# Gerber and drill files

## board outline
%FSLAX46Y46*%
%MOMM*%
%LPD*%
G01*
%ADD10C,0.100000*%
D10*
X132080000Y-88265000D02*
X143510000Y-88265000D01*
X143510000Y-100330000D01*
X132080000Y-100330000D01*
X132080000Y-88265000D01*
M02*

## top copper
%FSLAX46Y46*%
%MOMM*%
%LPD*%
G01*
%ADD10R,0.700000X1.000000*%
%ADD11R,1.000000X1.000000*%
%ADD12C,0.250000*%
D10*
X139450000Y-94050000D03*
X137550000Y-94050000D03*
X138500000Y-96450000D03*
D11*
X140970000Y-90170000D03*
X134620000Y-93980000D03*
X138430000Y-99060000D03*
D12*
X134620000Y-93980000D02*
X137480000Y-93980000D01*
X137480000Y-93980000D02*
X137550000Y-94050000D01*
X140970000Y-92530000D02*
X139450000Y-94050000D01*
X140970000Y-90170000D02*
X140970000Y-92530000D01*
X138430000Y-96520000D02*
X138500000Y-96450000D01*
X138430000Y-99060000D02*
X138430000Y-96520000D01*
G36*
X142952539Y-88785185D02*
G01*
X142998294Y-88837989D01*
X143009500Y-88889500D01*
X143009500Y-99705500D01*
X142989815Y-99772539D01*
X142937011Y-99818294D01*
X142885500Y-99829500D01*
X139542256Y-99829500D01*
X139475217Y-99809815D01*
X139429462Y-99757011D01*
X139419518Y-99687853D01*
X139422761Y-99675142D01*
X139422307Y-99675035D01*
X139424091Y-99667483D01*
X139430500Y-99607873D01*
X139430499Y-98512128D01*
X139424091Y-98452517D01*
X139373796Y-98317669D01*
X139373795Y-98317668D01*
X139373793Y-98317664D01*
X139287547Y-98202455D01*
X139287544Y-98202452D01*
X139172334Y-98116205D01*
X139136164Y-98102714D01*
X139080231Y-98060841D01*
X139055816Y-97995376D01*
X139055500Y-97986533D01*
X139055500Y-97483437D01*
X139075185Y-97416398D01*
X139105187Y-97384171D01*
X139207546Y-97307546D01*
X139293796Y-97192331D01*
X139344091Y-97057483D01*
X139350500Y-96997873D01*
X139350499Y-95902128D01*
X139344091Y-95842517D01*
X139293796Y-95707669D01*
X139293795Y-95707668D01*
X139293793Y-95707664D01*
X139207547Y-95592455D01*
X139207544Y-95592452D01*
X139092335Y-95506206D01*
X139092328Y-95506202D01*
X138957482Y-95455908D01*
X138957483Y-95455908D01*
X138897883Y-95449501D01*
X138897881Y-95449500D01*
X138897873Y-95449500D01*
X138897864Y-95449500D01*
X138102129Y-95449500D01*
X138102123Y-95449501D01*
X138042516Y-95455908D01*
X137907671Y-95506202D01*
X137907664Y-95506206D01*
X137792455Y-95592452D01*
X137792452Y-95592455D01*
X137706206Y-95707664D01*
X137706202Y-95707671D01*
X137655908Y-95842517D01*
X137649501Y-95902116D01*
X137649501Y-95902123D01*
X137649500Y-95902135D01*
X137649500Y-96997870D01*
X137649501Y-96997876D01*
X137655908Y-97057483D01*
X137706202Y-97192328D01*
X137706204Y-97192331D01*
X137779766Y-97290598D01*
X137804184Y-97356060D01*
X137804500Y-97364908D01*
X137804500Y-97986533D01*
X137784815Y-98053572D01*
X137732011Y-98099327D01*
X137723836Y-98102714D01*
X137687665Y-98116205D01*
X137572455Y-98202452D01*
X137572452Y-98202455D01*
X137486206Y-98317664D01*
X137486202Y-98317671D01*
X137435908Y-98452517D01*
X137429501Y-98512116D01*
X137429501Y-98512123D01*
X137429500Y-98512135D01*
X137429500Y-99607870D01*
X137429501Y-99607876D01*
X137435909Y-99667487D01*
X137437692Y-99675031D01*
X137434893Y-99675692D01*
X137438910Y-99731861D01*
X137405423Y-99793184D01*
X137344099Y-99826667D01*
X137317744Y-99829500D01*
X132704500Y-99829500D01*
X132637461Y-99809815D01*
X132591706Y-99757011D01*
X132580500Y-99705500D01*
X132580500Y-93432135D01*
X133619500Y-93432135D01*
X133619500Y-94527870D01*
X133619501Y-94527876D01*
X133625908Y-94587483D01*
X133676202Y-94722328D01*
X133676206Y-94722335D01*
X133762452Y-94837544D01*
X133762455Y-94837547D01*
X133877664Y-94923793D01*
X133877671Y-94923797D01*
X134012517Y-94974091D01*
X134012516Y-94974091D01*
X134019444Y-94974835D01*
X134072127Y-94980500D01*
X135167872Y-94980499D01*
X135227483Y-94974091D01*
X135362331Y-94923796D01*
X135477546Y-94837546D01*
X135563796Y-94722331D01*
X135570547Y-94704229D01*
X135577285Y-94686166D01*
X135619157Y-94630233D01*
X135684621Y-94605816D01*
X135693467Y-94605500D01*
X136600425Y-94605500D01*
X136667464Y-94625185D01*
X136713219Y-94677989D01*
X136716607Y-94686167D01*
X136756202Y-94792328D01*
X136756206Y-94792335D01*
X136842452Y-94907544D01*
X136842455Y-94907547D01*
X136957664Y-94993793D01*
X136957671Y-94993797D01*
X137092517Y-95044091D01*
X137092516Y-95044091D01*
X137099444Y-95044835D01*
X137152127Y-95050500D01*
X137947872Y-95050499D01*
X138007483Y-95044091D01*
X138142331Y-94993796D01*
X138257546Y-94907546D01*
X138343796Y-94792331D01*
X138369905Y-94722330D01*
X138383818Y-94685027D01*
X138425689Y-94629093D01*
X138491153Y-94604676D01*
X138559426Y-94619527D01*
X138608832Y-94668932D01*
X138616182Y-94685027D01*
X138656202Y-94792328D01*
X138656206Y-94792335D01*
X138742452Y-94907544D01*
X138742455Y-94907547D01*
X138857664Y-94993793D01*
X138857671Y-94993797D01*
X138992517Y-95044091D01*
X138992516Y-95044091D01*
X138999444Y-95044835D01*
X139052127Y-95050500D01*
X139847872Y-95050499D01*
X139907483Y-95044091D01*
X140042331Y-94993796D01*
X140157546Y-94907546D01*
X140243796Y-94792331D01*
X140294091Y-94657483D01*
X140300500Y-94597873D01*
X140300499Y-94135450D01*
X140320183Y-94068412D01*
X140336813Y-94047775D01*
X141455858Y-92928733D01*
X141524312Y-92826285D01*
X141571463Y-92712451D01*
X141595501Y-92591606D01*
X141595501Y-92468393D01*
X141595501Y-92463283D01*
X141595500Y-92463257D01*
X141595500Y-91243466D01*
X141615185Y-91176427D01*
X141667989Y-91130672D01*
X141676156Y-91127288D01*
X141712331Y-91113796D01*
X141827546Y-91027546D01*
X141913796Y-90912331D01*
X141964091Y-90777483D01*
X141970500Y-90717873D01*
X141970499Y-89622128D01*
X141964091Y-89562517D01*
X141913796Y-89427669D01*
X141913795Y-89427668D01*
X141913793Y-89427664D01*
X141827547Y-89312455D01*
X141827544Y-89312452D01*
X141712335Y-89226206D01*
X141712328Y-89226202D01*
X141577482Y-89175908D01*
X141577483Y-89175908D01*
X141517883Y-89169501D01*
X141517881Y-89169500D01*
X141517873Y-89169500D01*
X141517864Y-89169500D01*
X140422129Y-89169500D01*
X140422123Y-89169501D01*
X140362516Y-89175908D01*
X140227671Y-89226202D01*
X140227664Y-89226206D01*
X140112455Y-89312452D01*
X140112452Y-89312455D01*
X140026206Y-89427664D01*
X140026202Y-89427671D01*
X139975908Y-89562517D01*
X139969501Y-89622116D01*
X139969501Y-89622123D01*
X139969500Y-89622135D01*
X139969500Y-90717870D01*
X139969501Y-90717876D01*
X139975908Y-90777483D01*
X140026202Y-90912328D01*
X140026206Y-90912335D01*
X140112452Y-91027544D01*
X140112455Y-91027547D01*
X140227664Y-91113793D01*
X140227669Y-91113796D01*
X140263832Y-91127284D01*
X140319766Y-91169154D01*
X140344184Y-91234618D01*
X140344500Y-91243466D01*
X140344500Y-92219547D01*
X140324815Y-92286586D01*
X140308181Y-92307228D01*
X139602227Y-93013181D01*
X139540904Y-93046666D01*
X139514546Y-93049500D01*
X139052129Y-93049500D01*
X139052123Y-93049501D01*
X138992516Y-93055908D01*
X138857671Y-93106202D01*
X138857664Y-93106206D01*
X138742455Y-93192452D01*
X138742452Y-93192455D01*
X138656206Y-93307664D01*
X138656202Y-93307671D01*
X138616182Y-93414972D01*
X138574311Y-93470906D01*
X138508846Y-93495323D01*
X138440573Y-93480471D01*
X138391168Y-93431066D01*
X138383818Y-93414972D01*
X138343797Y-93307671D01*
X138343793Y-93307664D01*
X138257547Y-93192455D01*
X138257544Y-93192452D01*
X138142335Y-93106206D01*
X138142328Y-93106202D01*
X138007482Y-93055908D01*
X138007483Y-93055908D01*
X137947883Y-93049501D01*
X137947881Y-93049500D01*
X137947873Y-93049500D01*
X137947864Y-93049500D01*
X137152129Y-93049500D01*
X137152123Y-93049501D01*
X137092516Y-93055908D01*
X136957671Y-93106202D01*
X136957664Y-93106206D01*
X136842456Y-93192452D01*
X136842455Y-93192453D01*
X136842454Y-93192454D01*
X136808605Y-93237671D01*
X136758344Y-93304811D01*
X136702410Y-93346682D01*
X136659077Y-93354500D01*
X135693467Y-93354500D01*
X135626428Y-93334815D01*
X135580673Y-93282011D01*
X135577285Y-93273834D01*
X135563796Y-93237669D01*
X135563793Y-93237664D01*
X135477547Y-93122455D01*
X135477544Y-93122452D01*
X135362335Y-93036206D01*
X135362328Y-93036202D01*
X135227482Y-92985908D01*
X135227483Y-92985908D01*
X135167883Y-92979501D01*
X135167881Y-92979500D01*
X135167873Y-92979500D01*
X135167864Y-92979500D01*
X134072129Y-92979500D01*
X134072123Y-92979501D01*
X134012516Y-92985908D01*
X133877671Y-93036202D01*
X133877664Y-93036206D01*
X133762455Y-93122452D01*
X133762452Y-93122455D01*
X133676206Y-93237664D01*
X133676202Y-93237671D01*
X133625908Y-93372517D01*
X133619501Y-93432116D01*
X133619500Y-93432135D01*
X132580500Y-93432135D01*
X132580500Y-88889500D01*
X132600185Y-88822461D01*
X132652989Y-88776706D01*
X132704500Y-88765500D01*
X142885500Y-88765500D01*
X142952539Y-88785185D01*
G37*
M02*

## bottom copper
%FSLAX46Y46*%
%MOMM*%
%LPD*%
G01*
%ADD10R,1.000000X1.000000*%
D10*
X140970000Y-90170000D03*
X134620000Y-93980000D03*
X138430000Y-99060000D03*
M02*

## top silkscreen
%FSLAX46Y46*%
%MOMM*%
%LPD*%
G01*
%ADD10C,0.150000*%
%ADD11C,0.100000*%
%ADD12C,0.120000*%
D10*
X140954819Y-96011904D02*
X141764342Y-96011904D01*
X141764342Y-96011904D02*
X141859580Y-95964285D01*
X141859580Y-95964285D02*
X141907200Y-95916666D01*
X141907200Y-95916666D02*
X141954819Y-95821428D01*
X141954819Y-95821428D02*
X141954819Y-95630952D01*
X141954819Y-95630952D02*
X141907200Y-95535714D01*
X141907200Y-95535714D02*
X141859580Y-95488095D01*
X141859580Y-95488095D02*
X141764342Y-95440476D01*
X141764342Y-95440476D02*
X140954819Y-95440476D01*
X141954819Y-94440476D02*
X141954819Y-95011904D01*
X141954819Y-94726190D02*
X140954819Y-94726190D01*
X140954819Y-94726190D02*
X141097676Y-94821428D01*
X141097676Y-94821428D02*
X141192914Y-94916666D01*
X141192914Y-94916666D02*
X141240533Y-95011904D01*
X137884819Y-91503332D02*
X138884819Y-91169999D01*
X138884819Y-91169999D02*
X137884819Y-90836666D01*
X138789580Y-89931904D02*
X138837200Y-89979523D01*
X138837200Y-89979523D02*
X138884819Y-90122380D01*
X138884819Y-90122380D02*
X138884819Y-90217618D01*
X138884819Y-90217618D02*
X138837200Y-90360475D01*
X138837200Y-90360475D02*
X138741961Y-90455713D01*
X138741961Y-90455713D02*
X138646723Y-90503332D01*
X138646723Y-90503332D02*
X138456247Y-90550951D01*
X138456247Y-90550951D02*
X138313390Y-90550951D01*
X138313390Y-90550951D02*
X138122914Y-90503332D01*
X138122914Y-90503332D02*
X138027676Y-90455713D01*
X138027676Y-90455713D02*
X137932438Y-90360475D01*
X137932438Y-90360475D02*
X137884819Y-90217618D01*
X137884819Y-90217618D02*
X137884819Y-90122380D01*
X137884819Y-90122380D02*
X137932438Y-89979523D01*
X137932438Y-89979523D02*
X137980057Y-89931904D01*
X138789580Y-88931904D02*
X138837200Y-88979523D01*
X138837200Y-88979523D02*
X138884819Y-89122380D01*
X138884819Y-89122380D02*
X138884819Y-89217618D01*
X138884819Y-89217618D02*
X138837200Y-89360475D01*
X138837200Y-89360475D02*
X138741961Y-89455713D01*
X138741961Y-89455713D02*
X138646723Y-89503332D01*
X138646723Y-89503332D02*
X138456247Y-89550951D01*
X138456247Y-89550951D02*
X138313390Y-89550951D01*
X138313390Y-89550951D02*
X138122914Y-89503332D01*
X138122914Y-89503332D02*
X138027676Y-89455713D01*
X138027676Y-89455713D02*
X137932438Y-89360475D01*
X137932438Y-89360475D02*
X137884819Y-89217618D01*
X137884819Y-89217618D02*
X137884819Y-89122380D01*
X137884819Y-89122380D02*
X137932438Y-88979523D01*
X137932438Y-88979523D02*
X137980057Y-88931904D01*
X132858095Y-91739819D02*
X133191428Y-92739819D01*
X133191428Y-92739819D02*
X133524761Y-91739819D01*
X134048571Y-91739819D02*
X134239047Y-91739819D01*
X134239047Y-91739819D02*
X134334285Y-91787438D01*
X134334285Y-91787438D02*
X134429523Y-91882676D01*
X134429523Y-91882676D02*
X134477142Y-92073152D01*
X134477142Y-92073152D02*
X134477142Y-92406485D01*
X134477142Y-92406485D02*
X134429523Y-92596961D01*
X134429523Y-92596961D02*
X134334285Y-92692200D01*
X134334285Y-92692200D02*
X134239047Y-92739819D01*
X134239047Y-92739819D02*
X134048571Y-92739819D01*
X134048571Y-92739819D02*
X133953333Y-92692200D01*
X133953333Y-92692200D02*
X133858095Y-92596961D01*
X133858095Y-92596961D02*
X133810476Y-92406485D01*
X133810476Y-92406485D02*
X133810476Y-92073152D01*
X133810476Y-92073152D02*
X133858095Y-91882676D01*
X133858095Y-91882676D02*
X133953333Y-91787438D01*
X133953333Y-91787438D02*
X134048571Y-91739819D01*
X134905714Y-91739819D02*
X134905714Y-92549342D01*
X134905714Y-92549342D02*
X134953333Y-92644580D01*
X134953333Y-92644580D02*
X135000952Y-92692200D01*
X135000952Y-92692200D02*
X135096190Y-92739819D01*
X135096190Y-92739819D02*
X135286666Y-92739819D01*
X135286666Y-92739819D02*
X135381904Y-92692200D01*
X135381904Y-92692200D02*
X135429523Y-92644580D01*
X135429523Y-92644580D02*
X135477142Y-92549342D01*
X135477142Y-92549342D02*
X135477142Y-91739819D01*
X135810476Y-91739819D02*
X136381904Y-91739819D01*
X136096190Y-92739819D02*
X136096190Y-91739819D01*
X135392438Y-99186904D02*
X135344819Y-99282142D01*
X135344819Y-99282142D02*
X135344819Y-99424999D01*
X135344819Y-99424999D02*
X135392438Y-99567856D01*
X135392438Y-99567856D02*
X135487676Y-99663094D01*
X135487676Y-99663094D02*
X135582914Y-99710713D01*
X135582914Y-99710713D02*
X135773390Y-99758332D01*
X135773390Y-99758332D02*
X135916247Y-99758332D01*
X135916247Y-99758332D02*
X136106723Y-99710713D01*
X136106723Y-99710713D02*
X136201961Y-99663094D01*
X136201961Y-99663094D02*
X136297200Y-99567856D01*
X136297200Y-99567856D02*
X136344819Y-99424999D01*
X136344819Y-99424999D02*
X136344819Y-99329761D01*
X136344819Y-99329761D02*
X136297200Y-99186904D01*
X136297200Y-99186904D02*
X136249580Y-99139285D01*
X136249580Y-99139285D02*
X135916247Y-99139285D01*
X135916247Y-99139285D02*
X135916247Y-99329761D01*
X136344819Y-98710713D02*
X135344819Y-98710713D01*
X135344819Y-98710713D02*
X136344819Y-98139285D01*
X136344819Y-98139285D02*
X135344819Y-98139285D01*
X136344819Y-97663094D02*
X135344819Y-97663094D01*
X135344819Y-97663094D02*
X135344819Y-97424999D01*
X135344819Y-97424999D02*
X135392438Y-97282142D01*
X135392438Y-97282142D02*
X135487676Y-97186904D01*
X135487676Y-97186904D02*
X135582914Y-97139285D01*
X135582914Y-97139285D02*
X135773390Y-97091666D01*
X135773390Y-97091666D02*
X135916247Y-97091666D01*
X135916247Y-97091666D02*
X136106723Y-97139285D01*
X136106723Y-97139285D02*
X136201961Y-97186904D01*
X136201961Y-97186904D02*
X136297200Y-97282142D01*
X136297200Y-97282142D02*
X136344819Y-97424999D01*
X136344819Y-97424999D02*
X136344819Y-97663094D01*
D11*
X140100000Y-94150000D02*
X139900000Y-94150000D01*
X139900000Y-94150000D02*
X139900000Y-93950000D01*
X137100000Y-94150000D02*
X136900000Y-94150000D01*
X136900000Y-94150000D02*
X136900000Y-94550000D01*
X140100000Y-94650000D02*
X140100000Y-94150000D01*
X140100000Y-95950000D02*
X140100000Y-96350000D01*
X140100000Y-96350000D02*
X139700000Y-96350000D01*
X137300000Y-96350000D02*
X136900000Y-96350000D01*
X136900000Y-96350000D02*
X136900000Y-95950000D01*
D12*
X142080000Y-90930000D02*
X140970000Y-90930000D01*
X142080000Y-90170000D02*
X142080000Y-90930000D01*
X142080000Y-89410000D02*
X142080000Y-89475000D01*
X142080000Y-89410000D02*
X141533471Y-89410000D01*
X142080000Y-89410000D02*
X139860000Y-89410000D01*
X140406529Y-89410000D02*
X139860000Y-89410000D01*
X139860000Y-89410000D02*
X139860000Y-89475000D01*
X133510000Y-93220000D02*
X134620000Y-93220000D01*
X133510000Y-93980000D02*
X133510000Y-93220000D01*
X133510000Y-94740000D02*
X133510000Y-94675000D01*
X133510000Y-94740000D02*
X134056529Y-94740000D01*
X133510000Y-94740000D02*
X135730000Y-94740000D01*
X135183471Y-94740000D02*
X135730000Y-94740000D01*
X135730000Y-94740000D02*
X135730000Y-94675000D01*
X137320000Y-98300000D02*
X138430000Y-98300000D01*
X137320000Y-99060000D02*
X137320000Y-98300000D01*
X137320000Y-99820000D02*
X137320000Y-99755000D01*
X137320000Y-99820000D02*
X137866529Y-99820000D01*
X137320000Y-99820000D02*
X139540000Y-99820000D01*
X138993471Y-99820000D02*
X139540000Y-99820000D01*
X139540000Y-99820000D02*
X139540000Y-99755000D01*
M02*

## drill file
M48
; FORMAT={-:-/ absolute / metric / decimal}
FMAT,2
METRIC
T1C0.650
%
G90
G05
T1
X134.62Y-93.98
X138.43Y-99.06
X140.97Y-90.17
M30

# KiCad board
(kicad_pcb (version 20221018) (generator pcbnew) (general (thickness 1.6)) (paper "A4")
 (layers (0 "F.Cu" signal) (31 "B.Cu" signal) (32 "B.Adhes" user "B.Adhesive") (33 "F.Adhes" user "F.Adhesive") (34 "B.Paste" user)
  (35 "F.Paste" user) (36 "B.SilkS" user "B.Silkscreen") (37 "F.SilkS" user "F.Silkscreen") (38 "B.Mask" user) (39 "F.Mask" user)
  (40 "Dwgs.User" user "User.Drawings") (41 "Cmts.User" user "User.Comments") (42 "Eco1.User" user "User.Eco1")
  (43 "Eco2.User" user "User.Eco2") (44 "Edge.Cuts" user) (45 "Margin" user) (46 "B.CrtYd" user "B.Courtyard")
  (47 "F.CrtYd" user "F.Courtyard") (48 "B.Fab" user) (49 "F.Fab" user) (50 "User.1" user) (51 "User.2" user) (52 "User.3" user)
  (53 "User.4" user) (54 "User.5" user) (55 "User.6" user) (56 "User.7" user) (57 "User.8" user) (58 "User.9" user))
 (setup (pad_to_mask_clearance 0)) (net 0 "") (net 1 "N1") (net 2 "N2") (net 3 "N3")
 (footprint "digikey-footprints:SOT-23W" (layer "F.Cu") (at 138.5 95.25 -90)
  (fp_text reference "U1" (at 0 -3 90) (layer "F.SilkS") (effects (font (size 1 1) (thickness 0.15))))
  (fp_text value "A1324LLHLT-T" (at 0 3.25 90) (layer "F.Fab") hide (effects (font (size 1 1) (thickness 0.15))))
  (fp_line (start -1.1 -1.6) (end -1.1 -1.4) (stroke (width 0.1) (type solid)) (layer "F.SilkS"))
  (fp_line (start -1.1 -1.4) (end -1.3 -1.4) (stroke (width 0.1) (type solid)) (layer "F.SilkS"))
  (fp_line (start -1.1 1.4) (end -1.1 1.6) (stroke (width 0.1) (type solid)) (layer "F.SilkS"))
  (fp_line (start -1.1 1.6) (end -0.7 1.6) (stroke (width 0.1) (type solid)) (layer "F.SilkS"))
  (fp_line (start -0.6 -1.6) (end -1.1 -1.6) (stroke (width 0.1) (type solid)) (layer "F.SilkS"))
  (fp_line (start 0.7 -1.6) (end 1.1 -1.6) (stroke (width 0.1) (type solid)) (layer "F.SilkS"))
  (fp_line (start 1.1 -1.6) (end 1.1 -1.2) (stroke (width 0.1) (type solid)) (layer "F.SilkS"))
  (fp_line (start 1.1 1.2) (end 1.1 1.6) (stroke (width 0.1) (type solid)) (layer "F.SilkS"))
  (fp_line (start 1.1 1.6) (end 0.7 1.6) (stroke (width 0.1) (type solid)) (layer "F.SilkS"))
  (pad "1" smd rect (at -1.2 -0.95 270) (size 1 0.7) (layers "F.Cu" "F.Paste" "F.Mask") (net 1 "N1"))
  (pad "2" smd rect (at -1.2 0.95 270) (size 1 0.7) (layers "F.Cu" "F.Paste" "F.Mask") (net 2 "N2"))
  (pad "3" smd rect (at 1.2 0 270) (size 1 0.7) (layers "F.Cu" "F.Paste" "F.Mask") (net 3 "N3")))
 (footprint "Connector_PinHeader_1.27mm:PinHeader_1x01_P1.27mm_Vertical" (layer "F.Cu") (at 140.97 90.17 180)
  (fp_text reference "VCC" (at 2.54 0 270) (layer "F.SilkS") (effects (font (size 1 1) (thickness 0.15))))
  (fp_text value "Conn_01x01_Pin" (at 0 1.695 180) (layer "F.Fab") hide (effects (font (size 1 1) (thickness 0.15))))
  (fp_line (start -1.11 -0.76) (end 0 -0.76) (stroke (width 0.12) (type solid)) (layer "F.SilkS"))
  (fp_line (start -1.11 0) (end -1.11 -0.76) (stroke (width 0.12) (type solid)) (layer "F.SilkS"))
  (fp_line (start -1.11 0.76) (end -1.11 0.695) (stroke (width 0.12) (type solid)) (layer "F.SilkS"))
  (fp_line (start -1.11 0.76) (end -0.563471 0.76) (stroke (width 0.12) (type solid)) (layer "F.SilkS"))
  (fp_line (start -1.11 0.76) (end 1.11 0.76) (stroke (width 0.12) (type solid)) (layer "F.SilkS"))
  (fp_line (start 0.563471 0.76) (end 1.11 0.76) (stroke (width 0.12) (type solid)) (layer "F.SilkS"))
  (fp_line (start 1.11 0.76) (end 1.11 0.695) (stroke (width 0.12) (type solid)) (layer "F.SilkS"))
  (pad "1" thru_hole rect (at 0 0 180) (size 1 1) (drill 0.65) (layers "*.Cu" "*.Mask") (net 1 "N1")))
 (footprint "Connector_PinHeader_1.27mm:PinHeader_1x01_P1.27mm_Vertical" (layer "F.Cu") (at 134.62 93.98)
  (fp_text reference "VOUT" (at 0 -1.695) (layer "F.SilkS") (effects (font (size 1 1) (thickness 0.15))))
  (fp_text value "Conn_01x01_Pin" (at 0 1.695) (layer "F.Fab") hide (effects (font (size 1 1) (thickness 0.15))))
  (fp_line (start -1.11 -0.76) (end 0 -0.76) (stroke (width 0.12) (type solid)) (layer "F.SilkS"))
  (fp_line (start -1.11 0) (end -1.11 -0.76) (stroke (width 0.12) (type solid)) (layer "F.SilkS"))
  (fp_line (start -1.11 0.76) (end -1.11 0.695) (stroke (width 0.12) (type solid)) (layer "F.SilkS"))
  (fp_line (start -1.11 0.76) (end -0.563471 0.76) (stroke (width 0.12) (type solid)) (layer "F.SilkS"))
  (fp_line (start -1.11 0.76) (end 1.11 0.76) (stroke (width 0.12) (type solid)) (layer "F.SilkS"))
  (fp_line (start 0.563471 0.76) (end 1.11 0.76) (stroke (width 0.12) (type solid)) (layer "F.SilkS"))
  (fp_line (start 1.11 0.76) (end 1.11 0.695) (stroke (width 0.12) (type solid)) (layer "F.SilkS"))
  (pad "1" thru_hole rect (at 0 0) (size 1 1) (drill 0.65) (layers "*.Cu" "*.Mask") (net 2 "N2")))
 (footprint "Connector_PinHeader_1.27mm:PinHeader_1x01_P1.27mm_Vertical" (layer "F.Cu") (at 138.43 99.06)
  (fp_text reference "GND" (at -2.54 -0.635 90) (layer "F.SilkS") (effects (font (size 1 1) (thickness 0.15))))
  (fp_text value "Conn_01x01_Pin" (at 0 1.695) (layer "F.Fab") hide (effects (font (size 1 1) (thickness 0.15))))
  (fp_line (start -1.11 -0.76) (end 0 -0.76) (stroke (width 0.12) (type solid)) (layer "F.SilkS"))
  (fp_line (start -1.11 0) (end -1.11 -0.76) (stroke (width 0.12) (type solid)) (layer "F.SilkS"))
  (fp_line (start -1.11 0.76) (end -1.11 0.695) (stroke (width 0.12) (type solid)) (layer "F.SilkS"))
  (fp_line (start -1.11 0.76) (end -0.563471 0.76) (stroke (width 0.12) (type solid)) (layer "F.SilkS"))
  (fp_line (start -1.11 0.76) (end 1.11 0.76) (stroke (width 0.12) (type solid)) (layer "F.SilkS"))
  (fp_line (start 0.563471 0.76) (end 1.11 0.76) (stroke (width 0.12) (type solid)) (layer "F.SilkS"))
  (fp_line (start 1.11 0.76) (end 1.11 0.695) (stroke (width 0.12) (type solid)) (layer "F.SilkS"))
  (pad "1" thru_hole rect (at 0 0) (size 1 1) (drill 0.65) (layers "*.Cu" "*.Mask") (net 3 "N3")))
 (gr_poly
  (pts (xy 132.08 88.265) (xy 143.51 88.265) (xy 143.51 100.33) (xy 132.08 100.33)) (stroke (width 0.1) (type solid)) (fill none)
  (layer "Edge.Cuts"))
 (segment (start 134.62 93.98) (end 137.48 93.98) (width 0.25) (layer "F.Cu") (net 2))
 (segment (start 137.48 93.98) (end 137.55 94.05) (width 0.25) (layer "F.Cu") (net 2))
 (segment (start 140.97 92.53) (end 139.45 94.05) (width 0.25) (layer "F.Cu") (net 1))
 (segment (start 140.97 90.17) (end 140.97 92.53) (width 0.25) (layer "F.Cu") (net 1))
 (segment (start 138.43 96.52) (end 138.5 96.45) (width 0.25) (layer "F.Cu") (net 3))
 (segment (start 138.43 99.06) (end 138.43 96.52) (width 0.25) (layer "F.Cu") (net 3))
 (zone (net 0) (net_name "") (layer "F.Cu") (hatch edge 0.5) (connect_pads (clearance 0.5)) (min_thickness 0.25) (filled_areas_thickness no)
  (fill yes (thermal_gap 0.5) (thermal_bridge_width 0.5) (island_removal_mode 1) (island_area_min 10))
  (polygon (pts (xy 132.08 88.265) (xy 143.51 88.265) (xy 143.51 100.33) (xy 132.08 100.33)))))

